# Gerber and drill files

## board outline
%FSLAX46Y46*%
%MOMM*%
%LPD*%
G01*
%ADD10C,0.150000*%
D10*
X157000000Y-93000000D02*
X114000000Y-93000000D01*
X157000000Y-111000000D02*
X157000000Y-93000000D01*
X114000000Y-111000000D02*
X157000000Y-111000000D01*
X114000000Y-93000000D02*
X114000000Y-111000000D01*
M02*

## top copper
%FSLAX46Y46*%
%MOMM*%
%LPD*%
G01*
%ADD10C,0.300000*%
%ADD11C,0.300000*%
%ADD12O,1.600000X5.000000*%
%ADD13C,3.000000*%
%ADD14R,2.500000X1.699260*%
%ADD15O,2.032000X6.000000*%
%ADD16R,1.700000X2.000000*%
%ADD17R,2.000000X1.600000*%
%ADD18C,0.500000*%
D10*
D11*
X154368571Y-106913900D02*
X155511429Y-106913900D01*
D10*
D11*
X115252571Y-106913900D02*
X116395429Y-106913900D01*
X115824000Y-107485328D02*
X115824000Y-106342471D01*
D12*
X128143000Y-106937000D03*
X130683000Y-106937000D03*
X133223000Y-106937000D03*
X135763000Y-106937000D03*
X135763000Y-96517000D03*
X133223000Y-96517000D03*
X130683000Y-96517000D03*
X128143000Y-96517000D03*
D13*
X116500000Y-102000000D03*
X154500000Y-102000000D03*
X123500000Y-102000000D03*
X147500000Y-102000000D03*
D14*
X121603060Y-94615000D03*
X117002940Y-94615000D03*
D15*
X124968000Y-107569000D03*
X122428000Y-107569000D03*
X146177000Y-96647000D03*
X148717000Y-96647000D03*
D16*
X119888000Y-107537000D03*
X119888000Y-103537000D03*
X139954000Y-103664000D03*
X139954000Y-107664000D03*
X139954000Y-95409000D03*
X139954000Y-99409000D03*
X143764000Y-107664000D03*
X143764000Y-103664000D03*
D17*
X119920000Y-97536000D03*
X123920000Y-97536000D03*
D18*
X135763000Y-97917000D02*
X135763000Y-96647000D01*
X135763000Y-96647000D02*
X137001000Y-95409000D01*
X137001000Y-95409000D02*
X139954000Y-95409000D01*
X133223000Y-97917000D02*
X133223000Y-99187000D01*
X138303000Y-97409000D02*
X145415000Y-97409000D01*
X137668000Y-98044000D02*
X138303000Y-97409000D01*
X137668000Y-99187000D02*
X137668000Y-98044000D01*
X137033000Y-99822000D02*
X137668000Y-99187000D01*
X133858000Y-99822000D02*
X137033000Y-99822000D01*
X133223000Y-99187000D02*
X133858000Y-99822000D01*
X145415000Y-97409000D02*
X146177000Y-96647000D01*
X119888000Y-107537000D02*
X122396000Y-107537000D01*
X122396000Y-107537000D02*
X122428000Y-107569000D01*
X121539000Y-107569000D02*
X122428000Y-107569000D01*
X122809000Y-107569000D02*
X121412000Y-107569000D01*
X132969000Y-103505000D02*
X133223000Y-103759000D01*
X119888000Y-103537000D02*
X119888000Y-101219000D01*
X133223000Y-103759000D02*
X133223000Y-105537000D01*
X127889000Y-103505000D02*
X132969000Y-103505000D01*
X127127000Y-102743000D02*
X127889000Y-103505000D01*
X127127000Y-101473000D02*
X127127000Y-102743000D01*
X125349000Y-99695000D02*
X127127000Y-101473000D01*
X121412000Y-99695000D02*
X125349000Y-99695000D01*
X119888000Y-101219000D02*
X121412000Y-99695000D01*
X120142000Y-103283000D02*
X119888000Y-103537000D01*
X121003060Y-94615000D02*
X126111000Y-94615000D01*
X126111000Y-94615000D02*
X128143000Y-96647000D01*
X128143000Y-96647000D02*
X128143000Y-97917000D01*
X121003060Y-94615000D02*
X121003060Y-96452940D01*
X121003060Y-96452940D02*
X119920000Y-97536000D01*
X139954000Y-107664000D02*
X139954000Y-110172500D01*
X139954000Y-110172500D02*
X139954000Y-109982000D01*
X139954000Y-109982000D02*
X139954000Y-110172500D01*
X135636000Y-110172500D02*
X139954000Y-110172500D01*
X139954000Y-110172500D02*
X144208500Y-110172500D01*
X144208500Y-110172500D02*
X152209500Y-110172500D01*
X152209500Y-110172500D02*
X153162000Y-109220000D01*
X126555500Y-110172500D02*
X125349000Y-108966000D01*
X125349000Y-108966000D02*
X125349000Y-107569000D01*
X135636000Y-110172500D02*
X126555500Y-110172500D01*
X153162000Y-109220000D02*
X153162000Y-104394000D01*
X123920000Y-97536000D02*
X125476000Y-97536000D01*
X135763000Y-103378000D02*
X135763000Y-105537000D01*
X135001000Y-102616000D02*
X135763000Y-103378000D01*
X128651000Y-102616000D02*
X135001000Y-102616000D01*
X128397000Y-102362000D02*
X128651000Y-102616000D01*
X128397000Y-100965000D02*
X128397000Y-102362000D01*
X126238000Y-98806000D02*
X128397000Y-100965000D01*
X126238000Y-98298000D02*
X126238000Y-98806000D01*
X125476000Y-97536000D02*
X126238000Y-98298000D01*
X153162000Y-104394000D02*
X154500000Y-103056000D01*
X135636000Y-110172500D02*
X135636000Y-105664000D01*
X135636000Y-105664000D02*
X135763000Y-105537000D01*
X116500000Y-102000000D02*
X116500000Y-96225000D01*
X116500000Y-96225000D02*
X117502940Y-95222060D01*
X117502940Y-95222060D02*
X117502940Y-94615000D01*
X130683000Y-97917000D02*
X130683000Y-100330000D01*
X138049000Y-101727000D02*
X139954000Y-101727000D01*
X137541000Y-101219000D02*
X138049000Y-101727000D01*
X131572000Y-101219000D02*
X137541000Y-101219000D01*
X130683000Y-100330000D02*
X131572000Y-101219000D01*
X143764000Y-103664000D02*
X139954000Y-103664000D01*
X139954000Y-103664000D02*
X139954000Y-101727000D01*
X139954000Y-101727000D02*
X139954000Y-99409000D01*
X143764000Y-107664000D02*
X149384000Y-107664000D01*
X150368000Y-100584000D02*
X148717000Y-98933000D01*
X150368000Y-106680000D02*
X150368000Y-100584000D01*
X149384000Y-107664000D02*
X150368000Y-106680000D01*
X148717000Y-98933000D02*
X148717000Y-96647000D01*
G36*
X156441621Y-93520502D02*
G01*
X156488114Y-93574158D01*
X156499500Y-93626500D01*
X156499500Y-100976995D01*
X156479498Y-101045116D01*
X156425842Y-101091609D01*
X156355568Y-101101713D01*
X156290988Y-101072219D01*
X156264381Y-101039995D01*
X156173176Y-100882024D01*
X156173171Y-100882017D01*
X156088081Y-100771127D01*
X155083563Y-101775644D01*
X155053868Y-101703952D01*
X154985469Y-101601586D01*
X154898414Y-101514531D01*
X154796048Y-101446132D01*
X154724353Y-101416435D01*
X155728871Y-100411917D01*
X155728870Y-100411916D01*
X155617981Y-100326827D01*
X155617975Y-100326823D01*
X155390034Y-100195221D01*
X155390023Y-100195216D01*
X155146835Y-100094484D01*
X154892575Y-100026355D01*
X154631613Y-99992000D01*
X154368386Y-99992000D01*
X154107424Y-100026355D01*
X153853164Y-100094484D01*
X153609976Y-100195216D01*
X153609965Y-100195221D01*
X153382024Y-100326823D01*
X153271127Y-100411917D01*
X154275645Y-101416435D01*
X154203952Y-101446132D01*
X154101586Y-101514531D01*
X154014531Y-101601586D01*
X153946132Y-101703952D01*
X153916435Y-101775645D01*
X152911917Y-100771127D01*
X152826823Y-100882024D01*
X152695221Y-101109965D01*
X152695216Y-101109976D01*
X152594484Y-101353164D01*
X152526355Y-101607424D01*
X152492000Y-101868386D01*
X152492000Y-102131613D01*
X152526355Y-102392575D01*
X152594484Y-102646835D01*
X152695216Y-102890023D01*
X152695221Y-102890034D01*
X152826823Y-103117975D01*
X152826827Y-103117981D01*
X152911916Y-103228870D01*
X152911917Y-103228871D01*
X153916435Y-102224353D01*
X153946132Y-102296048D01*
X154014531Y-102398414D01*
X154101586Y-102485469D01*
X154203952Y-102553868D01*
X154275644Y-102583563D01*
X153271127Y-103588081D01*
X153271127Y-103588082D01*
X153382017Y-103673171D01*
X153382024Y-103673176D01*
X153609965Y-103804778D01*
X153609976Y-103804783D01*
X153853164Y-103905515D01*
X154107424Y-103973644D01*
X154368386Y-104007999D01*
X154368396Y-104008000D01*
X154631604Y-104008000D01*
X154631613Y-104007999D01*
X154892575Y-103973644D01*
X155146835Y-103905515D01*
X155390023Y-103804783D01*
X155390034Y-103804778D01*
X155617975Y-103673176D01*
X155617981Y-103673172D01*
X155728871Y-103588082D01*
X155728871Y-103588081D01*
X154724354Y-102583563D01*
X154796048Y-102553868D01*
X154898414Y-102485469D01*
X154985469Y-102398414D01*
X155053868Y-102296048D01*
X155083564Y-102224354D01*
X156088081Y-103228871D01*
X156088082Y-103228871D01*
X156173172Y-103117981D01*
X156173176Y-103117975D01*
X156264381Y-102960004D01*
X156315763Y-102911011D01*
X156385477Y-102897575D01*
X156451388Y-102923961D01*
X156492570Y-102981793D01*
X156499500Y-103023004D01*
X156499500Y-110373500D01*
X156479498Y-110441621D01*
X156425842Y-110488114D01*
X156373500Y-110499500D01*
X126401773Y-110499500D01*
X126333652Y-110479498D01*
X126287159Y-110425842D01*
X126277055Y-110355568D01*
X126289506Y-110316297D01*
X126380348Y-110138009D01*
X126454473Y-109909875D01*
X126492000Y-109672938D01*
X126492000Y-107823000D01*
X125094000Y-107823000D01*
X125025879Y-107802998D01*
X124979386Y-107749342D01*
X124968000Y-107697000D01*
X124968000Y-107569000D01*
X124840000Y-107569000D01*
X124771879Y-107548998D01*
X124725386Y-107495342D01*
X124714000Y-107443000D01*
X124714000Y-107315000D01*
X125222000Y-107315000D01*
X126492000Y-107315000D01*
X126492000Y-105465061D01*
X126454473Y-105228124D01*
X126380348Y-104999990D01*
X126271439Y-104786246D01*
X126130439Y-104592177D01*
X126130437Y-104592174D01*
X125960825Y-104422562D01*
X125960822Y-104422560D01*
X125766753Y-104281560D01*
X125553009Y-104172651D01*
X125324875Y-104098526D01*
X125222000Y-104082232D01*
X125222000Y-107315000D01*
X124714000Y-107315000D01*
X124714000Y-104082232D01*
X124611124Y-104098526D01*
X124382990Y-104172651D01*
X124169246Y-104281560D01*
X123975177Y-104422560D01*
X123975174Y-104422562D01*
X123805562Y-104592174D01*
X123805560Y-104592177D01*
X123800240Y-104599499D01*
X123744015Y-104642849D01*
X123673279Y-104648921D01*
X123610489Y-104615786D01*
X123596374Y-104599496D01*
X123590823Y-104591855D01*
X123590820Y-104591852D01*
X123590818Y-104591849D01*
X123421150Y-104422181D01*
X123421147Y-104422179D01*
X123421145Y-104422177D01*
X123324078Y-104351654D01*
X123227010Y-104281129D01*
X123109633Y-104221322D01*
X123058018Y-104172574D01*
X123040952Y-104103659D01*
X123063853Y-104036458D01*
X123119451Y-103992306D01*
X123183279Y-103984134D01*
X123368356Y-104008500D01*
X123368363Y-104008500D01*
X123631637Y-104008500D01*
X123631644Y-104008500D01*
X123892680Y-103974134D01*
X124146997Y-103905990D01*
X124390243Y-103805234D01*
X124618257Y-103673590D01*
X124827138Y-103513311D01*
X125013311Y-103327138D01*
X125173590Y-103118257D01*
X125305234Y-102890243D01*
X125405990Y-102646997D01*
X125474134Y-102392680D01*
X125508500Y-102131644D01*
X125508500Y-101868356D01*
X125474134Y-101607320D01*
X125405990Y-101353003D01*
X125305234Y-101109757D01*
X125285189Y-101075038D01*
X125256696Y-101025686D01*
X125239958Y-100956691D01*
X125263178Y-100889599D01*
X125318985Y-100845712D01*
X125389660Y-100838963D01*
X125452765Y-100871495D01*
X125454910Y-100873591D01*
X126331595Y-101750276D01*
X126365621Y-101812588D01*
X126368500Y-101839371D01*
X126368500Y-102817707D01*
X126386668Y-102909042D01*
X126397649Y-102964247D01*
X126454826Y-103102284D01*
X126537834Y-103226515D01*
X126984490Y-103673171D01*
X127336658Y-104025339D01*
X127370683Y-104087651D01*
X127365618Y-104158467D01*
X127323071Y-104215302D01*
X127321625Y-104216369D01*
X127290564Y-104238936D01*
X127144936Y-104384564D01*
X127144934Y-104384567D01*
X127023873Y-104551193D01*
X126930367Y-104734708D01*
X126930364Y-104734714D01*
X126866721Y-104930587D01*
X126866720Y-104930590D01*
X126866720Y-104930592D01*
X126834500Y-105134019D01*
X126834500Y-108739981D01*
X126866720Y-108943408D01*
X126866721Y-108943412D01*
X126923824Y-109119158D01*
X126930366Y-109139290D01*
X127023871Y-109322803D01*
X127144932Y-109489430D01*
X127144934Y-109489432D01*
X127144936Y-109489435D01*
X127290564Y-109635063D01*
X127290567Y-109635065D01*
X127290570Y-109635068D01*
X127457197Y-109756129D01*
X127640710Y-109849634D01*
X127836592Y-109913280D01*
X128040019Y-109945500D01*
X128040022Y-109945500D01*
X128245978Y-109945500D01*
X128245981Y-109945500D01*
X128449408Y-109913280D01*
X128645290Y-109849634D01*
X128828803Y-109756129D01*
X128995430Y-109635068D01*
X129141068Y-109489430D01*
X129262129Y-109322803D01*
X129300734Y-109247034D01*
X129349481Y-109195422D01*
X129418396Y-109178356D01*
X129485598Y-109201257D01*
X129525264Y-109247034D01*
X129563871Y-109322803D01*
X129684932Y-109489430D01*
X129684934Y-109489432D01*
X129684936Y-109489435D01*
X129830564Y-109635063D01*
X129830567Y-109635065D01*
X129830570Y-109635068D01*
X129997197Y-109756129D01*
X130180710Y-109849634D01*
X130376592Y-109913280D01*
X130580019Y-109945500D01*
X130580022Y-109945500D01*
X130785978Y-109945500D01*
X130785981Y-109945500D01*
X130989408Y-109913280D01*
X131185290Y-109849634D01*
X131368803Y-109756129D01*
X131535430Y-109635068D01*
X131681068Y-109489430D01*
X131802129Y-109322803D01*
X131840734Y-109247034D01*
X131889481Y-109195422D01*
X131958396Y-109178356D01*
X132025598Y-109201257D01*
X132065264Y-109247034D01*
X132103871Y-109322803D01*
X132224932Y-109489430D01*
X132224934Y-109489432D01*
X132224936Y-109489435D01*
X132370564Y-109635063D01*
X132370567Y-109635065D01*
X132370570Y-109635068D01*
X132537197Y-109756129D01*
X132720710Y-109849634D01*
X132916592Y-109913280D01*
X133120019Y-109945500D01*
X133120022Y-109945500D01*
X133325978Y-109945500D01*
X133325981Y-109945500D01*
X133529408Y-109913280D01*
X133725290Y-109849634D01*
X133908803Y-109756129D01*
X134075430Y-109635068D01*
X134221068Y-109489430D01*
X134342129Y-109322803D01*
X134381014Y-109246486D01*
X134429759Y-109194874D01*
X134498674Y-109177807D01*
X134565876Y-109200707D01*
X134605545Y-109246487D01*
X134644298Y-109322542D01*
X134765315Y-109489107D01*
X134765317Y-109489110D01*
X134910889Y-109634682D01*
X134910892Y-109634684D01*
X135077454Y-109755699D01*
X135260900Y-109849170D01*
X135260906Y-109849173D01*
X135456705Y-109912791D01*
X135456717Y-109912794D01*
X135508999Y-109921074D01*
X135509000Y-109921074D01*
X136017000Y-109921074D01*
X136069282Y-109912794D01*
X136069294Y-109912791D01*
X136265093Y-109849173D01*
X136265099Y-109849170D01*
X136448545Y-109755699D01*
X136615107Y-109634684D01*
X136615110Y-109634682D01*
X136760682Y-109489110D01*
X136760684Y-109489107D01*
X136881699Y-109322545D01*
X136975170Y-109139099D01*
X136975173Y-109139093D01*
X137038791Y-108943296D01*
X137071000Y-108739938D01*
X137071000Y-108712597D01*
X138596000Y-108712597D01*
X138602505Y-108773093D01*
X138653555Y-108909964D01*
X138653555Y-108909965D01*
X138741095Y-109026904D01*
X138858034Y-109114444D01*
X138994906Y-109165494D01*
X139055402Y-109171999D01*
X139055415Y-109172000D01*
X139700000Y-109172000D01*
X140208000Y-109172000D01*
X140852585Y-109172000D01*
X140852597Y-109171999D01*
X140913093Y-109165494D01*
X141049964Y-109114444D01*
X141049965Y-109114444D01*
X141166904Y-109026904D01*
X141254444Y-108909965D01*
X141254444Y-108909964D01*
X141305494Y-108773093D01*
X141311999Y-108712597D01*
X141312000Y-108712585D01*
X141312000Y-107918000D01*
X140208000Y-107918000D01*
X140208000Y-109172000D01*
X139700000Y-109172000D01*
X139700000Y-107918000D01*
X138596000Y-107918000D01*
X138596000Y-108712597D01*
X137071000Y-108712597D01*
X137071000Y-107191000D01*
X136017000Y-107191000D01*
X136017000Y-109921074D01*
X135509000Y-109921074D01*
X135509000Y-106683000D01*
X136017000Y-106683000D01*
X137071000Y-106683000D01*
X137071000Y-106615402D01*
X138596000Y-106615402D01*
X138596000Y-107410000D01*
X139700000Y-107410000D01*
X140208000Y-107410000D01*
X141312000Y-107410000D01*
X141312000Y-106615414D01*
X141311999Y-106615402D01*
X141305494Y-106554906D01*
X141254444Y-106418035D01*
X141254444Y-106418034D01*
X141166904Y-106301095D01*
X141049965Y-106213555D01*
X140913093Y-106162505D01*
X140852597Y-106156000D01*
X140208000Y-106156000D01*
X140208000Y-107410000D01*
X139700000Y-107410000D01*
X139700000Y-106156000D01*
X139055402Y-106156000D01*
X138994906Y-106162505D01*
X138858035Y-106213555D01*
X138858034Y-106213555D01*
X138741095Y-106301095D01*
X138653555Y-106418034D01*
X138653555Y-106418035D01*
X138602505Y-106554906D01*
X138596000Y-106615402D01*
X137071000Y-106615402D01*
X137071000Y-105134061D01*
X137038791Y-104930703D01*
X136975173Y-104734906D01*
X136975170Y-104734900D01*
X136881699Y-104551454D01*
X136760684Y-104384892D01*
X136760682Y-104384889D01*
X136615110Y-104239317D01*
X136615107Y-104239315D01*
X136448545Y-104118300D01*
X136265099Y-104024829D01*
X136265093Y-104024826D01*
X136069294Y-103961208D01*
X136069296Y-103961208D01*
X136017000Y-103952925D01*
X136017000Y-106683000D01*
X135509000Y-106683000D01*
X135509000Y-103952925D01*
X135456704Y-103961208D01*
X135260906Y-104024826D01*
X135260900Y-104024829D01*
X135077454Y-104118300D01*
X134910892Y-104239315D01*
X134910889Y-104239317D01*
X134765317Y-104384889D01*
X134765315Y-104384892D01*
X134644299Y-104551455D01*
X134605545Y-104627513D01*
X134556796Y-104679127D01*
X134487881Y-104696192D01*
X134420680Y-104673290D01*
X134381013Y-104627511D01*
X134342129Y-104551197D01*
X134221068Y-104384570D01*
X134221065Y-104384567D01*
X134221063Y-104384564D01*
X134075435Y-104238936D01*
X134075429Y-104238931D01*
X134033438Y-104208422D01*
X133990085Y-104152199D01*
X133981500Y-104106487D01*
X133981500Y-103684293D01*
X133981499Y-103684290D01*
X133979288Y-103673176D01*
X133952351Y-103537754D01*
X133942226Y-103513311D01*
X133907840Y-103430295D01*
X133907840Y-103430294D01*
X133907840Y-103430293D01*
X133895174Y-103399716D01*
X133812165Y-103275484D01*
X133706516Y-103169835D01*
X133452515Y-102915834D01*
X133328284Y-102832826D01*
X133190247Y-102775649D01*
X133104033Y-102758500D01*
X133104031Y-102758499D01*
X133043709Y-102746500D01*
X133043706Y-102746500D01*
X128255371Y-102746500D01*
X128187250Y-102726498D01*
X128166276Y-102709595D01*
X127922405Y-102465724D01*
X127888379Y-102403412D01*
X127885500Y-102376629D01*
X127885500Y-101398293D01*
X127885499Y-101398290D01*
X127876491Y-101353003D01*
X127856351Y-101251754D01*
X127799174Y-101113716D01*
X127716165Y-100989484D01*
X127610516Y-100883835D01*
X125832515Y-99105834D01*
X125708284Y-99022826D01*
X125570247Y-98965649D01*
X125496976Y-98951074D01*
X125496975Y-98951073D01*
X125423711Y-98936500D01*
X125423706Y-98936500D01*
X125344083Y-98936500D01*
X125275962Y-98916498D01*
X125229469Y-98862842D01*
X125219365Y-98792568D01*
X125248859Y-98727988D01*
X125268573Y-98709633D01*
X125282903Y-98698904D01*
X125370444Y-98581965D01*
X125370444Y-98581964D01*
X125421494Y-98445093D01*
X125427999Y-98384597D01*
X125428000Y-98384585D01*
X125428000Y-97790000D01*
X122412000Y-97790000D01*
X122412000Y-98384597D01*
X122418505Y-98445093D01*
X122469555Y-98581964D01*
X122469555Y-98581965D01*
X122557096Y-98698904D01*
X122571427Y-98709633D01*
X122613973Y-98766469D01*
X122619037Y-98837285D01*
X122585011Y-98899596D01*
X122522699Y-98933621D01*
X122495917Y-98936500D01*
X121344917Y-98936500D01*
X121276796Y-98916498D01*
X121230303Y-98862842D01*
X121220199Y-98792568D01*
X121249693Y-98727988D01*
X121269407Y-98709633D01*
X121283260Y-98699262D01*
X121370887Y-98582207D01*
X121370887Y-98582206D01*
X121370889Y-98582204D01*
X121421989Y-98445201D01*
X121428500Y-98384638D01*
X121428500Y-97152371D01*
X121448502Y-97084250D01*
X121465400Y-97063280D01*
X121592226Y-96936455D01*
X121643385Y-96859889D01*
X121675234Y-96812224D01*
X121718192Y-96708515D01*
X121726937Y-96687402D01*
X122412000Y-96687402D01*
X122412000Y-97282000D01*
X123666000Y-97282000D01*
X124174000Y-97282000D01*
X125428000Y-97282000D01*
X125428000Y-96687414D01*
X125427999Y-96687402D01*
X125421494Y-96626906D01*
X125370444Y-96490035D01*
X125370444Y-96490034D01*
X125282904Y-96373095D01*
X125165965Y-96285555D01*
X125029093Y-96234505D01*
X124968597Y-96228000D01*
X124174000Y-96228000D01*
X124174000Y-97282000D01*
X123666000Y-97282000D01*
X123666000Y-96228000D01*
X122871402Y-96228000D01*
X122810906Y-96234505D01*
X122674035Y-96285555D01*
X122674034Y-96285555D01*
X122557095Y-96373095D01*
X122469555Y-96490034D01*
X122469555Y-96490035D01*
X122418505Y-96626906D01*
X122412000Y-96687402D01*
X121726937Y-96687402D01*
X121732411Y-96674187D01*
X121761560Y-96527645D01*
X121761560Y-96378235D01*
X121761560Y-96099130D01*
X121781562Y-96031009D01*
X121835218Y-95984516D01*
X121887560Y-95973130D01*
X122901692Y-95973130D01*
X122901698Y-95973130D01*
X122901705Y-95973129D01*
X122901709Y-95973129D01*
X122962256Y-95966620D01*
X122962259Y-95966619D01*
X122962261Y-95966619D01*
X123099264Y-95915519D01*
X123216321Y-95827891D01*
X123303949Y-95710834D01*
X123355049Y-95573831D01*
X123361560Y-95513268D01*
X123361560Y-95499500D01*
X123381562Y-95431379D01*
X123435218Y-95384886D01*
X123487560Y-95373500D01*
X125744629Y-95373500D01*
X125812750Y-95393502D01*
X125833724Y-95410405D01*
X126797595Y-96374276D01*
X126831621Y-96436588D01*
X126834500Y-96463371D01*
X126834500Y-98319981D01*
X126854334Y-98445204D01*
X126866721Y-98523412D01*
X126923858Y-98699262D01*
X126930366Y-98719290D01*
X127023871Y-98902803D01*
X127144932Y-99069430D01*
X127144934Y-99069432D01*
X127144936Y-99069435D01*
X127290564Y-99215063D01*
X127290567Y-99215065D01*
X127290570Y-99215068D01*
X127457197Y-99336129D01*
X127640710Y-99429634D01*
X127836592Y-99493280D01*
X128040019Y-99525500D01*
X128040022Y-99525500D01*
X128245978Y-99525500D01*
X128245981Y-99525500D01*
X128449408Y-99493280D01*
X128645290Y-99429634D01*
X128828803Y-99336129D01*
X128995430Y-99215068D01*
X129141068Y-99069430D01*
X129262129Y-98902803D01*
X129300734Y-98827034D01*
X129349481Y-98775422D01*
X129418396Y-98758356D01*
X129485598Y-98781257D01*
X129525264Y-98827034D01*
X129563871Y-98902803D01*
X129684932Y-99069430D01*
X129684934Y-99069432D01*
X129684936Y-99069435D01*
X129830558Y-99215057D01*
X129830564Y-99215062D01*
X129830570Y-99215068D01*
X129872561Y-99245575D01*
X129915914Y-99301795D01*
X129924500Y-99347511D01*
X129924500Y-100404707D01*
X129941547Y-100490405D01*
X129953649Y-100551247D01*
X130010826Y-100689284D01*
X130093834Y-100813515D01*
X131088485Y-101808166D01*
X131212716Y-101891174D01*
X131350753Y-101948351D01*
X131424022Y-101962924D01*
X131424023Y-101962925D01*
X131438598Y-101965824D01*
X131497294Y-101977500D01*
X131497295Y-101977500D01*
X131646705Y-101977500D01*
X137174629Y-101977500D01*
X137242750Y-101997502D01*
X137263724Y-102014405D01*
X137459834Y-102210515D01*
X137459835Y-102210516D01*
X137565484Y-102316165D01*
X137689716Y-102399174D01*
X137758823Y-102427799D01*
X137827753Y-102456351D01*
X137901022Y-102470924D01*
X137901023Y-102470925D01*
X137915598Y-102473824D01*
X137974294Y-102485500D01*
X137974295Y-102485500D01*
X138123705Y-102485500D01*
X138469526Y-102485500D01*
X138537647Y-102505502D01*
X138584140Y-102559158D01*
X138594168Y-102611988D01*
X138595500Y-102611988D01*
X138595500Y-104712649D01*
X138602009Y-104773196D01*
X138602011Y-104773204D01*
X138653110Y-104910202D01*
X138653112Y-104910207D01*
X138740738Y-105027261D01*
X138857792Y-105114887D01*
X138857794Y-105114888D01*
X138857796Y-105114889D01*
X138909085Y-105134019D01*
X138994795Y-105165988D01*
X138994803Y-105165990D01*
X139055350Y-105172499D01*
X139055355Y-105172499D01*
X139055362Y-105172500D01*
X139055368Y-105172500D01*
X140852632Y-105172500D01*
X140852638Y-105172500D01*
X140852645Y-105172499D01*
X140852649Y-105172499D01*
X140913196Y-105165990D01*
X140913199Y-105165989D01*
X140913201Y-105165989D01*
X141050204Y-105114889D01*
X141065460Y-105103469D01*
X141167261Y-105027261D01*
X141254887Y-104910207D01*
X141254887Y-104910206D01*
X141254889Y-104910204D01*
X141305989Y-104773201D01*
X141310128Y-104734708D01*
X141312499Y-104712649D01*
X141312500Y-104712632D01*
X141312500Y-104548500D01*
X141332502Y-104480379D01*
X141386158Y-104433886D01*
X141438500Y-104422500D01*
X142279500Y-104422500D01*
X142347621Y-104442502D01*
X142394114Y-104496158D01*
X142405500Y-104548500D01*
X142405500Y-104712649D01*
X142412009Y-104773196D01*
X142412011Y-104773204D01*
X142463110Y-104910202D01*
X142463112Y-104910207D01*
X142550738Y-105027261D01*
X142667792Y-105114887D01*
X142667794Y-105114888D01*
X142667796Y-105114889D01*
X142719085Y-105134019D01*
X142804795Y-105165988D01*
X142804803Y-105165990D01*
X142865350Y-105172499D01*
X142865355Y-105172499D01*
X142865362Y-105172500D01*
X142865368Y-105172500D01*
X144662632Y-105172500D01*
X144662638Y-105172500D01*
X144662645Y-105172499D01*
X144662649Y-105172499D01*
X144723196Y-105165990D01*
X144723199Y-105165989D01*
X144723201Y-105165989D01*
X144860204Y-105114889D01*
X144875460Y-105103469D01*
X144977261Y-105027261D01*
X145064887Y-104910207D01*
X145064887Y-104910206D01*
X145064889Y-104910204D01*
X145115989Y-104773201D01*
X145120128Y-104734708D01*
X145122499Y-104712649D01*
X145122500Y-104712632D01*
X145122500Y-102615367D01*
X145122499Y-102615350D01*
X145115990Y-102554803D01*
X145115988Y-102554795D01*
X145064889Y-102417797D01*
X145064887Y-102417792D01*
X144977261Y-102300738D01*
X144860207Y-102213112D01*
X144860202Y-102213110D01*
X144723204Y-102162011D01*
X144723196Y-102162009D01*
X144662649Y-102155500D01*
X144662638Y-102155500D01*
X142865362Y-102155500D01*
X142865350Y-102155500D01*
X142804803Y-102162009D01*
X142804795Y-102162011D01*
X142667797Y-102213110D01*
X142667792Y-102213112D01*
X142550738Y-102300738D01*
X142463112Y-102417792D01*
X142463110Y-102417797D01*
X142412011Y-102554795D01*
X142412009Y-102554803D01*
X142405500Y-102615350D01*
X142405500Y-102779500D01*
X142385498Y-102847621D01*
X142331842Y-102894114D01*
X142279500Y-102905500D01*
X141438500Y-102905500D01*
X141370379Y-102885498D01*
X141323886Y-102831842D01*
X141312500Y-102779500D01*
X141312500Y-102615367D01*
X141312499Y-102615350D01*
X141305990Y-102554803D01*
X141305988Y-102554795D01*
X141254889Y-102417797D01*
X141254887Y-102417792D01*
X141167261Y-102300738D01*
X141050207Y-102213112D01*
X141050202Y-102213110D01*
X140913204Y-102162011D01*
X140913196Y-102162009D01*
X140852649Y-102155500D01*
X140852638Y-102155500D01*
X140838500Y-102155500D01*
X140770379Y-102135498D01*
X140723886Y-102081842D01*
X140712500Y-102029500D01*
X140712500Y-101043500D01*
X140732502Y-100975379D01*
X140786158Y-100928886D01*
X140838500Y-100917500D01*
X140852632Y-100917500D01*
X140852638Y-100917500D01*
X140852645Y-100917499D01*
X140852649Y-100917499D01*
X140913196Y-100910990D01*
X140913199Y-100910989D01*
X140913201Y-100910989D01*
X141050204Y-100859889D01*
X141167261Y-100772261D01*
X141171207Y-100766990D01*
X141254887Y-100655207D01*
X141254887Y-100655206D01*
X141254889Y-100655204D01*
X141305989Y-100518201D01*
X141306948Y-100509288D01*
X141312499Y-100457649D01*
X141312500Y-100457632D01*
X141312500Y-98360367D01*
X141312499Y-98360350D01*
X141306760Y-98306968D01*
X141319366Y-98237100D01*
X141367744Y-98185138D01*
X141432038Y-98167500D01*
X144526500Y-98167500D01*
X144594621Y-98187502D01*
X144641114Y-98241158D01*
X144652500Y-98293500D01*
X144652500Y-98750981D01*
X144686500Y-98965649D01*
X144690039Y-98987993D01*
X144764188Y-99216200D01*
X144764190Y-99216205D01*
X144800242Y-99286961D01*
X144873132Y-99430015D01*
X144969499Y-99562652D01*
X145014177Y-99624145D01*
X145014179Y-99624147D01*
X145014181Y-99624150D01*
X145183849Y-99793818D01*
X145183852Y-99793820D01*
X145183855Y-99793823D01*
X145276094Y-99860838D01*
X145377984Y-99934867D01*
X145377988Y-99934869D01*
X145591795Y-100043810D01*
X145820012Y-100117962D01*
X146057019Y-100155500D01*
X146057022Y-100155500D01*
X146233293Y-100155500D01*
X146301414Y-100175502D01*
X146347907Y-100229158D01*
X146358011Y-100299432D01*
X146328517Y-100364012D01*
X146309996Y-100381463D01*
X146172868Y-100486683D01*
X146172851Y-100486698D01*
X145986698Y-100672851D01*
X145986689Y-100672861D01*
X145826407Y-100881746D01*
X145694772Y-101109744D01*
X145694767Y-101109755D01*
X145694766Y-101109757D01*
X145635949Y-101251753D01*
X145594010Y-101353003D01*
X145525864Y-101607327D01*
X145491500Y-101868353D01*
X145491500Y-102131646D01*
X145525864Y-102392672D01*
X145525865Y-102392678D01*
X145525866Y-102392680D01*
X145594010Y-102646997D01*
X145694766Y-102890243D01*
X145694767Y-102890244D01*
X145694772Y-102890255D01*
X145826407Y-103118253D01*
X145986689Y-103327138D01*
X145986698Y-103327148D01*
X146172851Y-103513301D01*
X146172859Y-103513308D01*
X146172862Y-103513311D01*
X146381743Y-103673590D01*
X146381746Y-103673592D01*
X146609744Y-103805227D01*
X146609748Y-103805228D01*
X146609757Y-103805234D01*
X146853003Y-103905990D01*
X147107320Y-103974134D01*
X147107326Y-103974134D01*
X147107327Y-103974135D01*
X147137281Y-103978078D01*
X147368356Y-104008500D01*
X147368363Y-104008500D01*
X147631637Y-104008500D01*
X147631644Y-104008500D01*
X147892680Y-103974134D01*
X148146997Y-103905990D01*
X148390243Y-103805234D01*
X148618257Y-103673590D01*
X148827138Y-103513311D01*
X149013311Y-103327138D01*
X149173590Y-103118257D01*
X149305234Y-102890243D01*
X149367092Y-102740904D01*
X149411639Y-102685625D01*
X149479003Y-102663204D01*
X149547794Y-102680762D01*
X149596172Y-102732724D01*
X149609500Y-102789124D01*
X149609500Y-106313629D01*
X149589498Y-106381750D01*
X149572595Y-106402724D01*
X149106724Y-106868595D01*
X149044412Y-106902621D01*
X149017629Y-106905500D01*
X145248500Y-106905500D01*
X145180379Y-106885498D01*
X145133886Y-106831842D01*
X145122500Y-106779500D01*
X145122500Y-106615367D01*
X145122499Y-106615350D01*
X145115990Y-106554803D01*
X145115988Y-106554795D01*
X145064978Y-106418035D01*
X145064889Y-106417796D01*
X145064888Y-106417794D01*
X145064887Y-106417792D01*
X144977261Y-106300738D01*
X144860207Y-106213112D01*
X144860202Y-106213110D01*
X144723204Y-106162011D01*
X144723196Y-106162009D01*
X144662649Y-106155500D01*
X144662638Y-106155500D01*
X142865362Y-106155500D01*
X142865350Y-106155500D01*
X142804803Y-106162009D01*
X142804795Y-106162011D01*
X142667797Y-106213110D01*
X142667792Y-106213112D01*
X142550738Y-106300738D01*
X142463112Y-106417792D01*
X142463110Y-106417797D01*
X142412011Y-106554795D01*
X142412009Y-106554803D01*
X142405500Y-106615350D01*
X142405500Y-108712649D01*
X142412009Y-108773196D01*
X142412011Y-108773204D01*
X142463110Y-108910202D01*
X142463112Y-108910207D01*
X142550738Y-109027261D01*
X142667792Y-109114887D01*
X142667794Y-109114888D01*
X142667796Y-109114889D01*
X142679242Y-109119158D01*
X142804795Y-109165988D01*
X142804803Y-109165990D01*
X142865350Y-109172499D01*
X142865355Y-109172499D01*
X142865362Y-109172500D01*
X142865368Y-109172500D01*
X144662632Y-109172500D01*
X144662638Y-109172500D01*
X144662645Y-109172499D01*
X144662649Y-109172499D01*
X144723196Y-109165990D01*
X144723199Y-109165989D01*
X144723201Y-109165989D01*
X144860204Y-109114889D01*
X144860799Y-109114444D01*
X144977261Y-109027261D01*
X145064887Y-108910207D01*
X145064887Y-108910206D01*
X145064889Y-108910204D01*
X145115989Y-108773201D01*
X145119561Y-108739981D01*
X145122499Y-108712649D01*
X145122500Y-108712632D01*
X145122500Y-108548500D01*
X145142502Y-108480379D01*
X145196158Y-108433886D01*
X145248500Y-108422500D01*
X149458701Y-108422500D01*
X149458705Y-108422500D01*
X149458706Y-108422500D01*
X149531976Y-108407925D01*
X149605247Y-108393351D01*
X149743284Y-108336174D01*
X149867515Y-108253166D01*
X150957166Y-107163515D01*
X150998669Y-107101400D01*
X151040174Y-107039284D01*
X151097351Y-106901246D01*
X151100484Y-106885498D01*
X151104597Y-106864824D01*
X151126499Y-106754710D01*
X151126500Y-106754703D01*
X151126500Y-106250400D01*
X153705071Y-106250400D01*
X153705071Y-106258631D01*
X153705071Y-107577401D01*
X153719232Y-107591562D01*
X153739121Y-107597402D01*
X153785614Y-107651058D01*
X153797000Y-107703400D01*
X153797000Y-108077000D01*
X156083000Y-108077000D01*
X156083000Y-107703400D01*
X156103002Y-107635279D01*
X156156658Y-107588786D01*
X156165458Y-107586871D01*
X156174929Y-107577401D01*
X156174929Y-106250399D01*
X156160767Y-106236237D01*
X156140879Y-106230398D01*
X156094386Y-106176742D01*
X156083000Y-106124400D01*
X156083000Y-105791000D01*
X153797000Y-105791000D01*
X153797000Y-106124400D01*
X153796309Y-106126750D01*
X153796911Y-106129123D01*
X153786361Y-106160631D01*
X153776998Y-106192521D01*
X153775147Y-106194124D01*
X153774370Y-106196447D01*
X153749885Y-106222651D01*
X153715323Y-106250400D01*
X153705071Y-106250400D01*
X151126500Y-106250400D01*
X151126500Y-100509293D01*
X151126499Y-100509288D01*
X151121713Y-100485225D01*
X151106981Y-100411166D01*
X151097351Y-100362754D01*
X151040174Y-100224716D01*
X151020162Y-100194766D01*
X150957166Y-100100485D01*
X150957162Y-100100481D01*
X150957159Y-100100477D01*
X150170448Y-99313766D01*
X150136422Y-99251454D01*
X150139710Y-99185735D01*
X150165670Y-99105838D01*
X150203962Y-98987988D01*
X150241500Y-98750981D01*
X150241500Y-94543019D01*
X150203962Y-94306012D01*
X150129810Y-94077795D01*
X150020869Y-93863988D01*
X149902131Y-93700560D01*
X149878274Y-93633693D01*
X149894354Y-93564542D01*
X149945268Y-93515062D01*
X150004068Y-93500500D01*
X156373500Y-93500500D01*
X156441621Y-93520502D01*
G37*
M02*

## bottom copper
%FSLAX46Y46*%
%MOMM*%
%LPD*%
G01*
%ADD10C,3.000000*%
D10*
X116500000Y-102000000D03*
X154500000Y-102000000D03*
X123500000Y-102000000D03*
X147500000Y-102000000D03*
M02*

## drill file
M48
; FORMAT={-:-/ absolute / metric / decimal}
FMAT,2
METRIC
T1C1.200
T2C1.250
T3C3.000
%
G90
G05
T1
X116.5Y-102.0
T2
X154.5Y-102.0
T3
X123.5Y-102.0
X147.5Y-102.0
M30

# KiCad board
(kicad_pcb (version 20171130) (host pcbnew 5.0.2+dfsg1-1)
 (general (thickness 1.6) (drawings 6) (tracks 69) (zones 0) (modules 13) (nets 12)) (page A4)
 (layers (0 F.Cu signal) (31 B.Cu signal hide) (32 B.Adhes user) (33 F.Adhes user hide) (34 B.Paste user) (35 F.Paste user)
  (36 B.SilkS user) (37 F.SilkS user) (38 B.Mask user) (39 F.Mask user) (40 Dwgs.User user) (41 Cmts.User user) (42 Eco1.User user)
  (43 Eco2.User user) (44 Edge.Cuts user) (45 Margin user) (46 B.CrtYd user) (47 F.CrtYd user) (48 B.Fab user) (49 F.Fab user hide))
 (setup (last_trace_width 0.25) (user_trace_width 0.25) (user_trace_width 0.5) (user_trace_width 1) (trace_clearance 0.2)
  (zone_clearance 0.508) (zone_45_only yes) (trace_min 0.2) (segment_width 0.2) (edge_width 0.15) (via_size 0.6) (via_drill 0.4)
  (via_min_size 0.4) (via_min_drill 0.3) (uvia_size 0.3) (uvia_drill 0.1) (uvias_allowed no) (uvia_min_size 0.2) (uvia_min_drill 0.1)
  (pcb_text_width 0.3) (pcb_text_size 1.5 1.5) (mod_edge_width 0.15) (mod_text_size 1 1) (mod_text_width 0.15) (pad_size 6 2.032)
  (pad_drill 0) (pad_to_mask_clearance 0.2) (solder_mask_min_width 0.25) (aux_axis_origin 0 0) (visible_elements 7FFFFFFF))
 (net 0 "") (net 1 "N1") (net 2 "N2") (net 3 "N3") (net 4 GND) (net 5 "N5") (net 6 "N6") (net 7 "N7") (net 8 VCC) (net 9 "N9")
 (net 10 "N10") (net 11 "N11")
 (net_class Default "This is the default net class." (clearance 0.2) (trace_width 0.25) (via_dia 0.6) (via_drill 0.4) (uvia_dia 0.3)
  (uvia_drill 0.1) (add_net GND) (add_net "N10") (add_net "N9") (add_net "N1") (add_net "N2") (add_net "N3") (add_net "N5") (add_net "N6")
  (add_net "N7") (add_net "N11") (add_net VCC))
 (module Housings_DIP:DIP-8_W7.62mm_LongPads (layer F.Cu) (at 128.143 105.537 90)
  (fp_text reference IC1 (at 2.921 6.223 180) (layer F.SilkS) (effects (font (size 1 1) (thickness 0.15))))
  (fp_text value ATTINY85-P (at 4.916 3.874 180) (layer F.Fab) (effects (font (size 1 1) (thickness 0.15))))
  (pad 1 smd oval (at 0 0 90) (size 5 1.6) (drill (offset -1.4 0)) (layers F.Cu F.Paste F.Mask) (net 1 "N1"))
  (pad 2 smd oval (at 0 2.54 90) (size 5 1.6) (drill (offset -1.4 0)) (layers F.Cu F.Paste F.Mask) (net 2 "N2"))
  (pad 3 smd oval (at 0 5.08 90) (size 5 1.6) (drill (offset -1.4 0)) (layers F.Cu F.Paste F.Mask) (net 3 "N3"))
  (pad 4 smd oval (at 0 7.62 90) (size 5 1.6) (drill (offset -1.4 0)) (layers F.Cu F.Paste F.Mask) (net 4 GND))
  (pad 5 smd oval (at 7.62 7.62 90) (size 5 1.6) (drill (offset 1.4 0)) (layers F.Cu F.Paste F.Mask) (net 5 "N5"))
  (pad 6 smd oval (at 7.62 5.08 90) (size 5 1.6) (drill (offset 1.4 0)) (layers F.Cu F.Paste F.Mask) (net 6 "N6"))
  (pad 7 smd oval (at 7.62 2.54 90) (size 5 1.6) (drill (offset 1.4 0)) (layers F.Cu F.Paste F.Mask) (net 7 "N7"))
  (pad 8 smd oval (at 7.62 0 90) (size 5 1.6) (drill (offset 1.4 0)) (layers F.Cu F.Paste F.Mask) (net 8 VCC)))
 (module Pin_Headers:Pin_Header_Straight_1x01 (layer F.Cu) (at 116.5 102)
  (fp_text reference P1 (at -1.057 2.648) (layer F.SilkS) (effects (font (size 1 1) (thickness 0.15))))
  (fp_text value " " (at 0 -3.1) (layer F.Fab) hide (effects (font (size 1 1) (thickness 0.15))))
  (pad 1 thru_hole circle (at 0 0) (size 3 3) (drill 1.2) (layers F.Cu F.SilkS F.Mask) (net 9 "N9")))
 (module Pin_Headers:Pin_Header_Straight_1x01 (layer F.Cu) (at 154.5 102)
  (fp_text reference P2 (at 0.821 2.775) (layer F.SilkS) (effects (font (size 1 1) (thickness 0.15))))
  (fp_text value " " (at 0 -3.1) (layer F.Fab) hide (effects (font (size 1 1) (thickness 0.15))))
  (pad 1 thru_hole circle (at 0 0) (size 3 3) (drill 1.25) (layers *.Mask F.Cu F.SilkS) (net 4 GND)))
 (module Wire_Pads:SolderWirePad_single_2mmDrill (layer F.Cu) (at 123.5 102)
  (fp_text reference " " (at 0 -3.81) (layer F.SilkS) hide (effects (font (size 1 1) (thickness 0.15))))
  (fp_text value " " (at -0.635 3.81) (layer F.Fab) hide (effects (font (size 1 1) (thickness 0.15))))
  (pad 1 thru_hole circle (at 0 0) (size 3 3) (drill 3) (layers *.Mask F.Cu F.SilkS)))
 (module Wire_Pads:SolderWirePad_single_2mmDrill (layer F.Cu) (at 147.5 102)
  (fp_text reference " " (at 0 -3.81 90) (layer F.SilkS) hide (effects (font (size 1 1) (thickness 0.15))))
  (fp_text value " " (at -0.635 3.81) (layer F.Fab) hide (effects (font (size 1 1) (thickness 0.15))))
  (pad 1 thru_hole circle (at 0 0) (size 3 3) (drill 3) (layers *.Mask F.Cu F.SilkS)))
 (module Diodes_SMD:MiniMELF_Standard (layer F.Cu) (at 119.253 94.615 180)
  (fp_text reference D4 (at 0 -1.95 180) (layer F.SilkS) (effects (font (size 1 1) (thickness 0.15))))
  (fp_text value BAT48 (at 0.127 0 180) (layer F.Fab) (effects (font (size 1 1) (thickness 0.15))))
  (pad 1 smd rect (at -1.75006 0 180) (size 2.5 1.69926) (drill (offset -0.6 0)) (layers F.Cu F.Paste F.Mask) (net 8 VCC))
  (pad 2 smd rect (at 1.75006 0 180) (size 2.5 1.69926) (drill (offset 0.5 0)) (layers F.Cu F.Paste F.Mask) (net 9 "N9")))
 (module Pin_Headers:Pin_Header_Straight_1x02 (layer F.Cu) (at 124.968 107.569 270)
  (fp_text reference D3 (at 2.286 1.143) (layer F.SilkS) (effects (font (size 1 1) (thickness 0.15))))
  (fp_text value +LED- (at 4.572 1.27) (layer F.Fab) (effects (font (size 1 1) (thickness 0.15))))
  (pad 1 smd oval (at 0 0 270) (size 6 2.032) (layers F.Cu F.Paste F.Mask) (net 4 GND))
  (pad 2 smd oval (at 0 2.54 270) (size 6 2.032) (layers F.Cu F.Paste F.Mask) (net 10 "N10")))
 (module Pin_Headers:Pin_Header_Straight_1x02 (layer F.Cu) (at 146.177 96.647 90)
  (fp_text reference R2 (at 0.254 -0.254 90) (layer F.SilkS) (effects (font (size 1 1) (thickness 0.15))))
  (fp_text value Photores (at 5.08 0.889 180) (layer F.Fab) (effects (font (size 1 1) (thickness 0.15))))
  (pad 1 smd oval (at 0 0 90) (size 6 2.032) (layers F.Cu F.Paste F.Mask) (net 6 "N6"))
  (pad 2 smd oval (at 0 2.54 90) (size 6 2.032) (layers F.Cu F.Paste F.Mask) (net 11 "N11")))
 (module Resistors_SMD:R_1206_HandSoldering (layer F.Cu) (at 119.888 105.537 90)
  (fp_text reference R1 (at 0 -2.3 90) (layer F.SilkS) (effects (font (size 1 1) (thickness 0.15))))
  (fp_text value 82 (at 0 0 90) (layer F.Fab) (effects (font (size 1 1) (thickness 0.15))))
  (pad 1 smd rect (at -2 0 90) (size 2 1.7) (layers F.Cu F.Paste F.Mask) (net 10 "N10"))
  (pad 2 smd rect (at 2 0 90) (size 2 1.7) (layers F.Cu F.Paste F.Mask) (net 3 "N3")))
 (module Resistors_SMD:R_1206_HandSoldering (layer F.Cu) (at 139.954 105.664 270)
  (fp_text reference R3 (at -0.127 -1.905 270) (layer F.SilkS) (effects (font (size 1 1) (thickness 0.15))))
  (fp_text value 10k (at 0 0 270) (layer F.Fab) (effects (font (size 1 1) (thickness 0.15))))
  (pad 1 smd rect (at -2 0 270) (size 2 1.7) (layers F.Cu F.Paste F.Mask) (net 7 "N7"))
  (pad 2 smd rect (at 2 0 270) (size 2 1.7) (layers F.Cu F.Paste F.Mask) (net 4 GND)))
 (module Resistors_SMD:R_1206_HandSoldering (layer F.Cu) (at 139.954 97.409 270)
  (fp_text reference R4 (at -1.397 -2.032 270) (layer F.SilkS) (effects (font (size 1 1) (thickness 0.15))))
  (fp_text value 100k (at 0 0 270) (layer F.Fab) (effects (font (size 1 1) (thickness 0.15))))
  (pad 1 smd rect (at -2 0 270) (size 2 1.7) (layers F.Cu F.Paste F.Mask) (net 5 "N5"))
  (pad 2 smd rect (at 2 0 270) (size 2 1.7) (layers F.Cu F.Paste F.Mask) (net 7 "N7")))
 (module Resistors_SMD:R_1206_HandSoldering (layer F.Cu) (at 143.764 105.664 90)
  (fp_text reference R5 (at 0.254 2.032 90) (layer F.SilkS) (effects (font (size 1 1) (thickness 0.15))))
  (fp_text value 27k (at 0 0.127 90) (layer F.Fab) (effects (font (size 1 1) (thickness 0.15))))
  (pad 1 smd rect (at -2 0 90) (size 2 1.7) (layers F.Cu F.Paste F.Mask) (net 11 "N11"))
  (pad 2 smd rect (at 2 0 90) (size 2 1.7) (layers F.Cu F.Paste F.Mask) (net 7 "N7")))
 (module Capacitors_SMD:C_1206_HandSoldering (layer F.Cu) (at 121.92 97.536)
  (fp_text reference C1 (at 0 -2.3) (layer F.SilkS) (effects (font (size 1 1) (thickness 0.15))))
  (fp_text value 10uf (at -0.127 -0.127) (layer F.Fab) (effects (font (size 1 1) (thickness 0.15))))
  (pad 1 smd rect (at -2 0) (size 2 1.6) (layers F.Cu F.Paste F.Mask) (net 8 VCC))
  (pad 2 smd rect (at 2 0) (size 2 1.6) (layers F.Cu F.Paste F.Mask) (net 4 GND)))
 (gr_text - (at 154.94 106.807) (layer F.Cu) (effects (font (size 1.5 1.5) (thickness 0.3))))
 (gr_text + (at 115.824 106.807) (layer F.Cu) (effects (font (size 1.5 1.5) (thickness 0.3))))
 (gr_line (start 157 93) (end 114 93) (angle 90) (layer Edge.Cuts) (width 0.15))
 (gr_line (start 157 111) (end 157 93) (angle 90) (layer Edge.Cuts) (width 0.15))
 (gr_line (start 114 111) (end 157 111) (angle 90) (layer Edge.Cuts) (width 0.15))
 (gr_line (start 114 93) (end 114 111) (angle 90) (layer Edge.Cuts) (width 0.15))
 (segment (start 135.763 97.917) (end 135.763 96.647) (width 0.5) (layer F.Cu) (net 5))
 (segment (start 135.763 96.647) (end 137.001 95.409) (width 0.5) (layer F.Cu) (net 5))
 (segment (start 137.001 95.409) (end 139.954 95.409) (width 0.5) (layer F.Cu) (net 5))
 (segment (start 133.223 97.917) (end 133.223 99.187) (width 0.5) (layer F.Cu) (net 6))
 (segment (start 138.303 97.409) (end 145.415 97.409) (width 0.5) (layer F.Cu) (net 6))
 (segment (start 137.668 98.044) (end 138.303 97.409) (width 0.5) (layer F.Cu) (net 6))
 (segment (start 137.668 99.187) (end 137.668 98.044) (width 0.5) (layer F.Cu) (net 6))
 (segment (start 137.033 99.822) (end 137.668 99.187) (width 0.5) (layer F.Cu) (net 6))
 (segment (start 133.858 99.822) (end 137.033 99.822) (width 0.5) (layer F.Cu) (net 6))
 (segment (start 133.223 99.187) (end 133.858 99.822) (width 0.5) (layer F.Cu) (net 6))
 (segment (start 145.415 97.409) (end 146.177 96.647) (width 0.5) (layer F.Cu) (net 6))
 (segment (start 119.888 107.537) (end 122.396 107.537) (width 0.5) (layer F.Cu) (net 10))
 (segment (start 122.396 107.537) (end 122.428 107.569) (width 0.5) (layer F.Cu) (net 10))
 (segment (start 121.539 107.569) (end 122.428 107.569) (width 0.5) (layer F.Cu) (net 10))
 (segment (start 122.809 107.569) (end 121.412 107.569) (width 0.5) (layer F.Cu) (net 10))
 (segment (start 132.969 103.505) (end 133.223 103.759) (width 0.5) (layer F.Cu) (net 3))
 (segment (start 119.888 103.537) (end 119.888 101.219) (width 0.5) (layer F.Cu) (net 3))
 (segment (start 133.223 103.759) (end 133.223 105.537) (width 0.5) (layer F.Cu) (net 3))
 (segment (start 127.889 103.505) (end 132.969 103.505) (width 0.5) (layer F.Cu) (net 3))
 (segment (start 127.127 102.743) (end 127.889 103.505) (width 0.5) (layer F.Cu) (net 3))
 (segment (start 127.127 101.473) (end 127.127 102.743) (width 0.5) (layer F.Cu) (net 3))
 (segment (start 125.349 99.695) (end 127.127 101.473) (width 0.5) (layer F.Cu) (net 3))
 (segment (start 121.412 99.695) (end 125.349 99.695) (width 0.5) (layer F.Cu) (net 3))
 (segment (start 119.888 101.219) (end 121.412 99.695) (width 0.5) (layer F.Cu) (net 3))
 (segment (start 120.142 103.283) (end 119.888 103.537) (width 0.5) (layer F.Cu) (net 3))
 (segment (start 121.00306 94.615) (end 126.111 94.615) (width 0.5) (layer F.Cu) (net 8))
 (segment (start 126.111 94.615) (end 128.143 96.647) (width 0.5) (layer F.Cu) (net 8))
 (segment (start 128.143 96.647) (end 128.143 97.917) (width 0.5) (layer F.Cu) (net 8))
 (segment (start 121.00306 94.615) (end 121.00306 96.45294) (width 0.5) (layer F.Cu) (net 8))
 (segment (start 121.00306 96.45294) (end 119.92 97.536) (width 0.5) (layer F.Cu) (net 8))
 (segment (start 139.954 107.664) (end 139.954 110.1725) (width 0.5) (layer F.Cu) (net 4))
 (segment (start 139.954 110.1725) (end 139.954 109.982) (width 0.5) (layer F.Cu) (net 4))
 (segment (start 139.954 109.982) (end 139.954 110.1725) (width 0.5) (layer F.Cu) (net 4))
 (segment (start 135.636 110.1725) (end 139.954 110.1725) (width 0.5) (layer F.Cu) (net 4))
 (segment (start 139.954 110.1725) (end 144.2085 110.1725) (width 0.5) (layer F.Cu) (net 4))
 (segment (start 144.2085 110.1725) (end 152.2095 110.1725) (width 0.5) (layer F.Cu) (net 4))
 (segment (start 152.2095 110.1725) (end 153.162 109.22) (width 0.5) (layer F.Cu) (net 4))
 (segment (start 126.5555 110.1725) (end 125.349 108.966) (width 0.5) (layer F.Cu) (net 4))
 (segment (start 125.349 108.966) (end 125.349 107.569) (width 0.5) (layer F.Cu) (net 4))
 (segment (start 135.636 110.1725) (end 126.5555 110.1725) (width 0.5) (layer F.Cu) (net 4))
 (segment (start 153.162 109.22) (end 153.162 104.394) (width 0.5) (layer F.Cu) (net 4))
 (segment (start 123.92 97.536) (end 125.476 97.536) (width 0.5) (layer F.Cu) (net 4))
 (segment (start 135.763 103.378) (end 135.763 105.537) (width 0.5) (layer F.Cu) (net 4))
 (segment (start 135.001 102.616) (end 135.763 103.378) (width 0.5) (layer F.Cu) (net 4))
 (segment (start 128.651 102.616) (end 135.001 102.616) (width 0.5) (layer F.Cu) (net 4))
 (segment (start 128.397 102.362) (end 128.651 102.616) (width 0.5) (layer F.Cu) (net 4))
 (segment (start 128.397 100.965) (end 128.397 102.362) (width 0.5) (layer F.Cu) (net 4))
 (segment (start 126.238 98.806) (end 128.397 100.965) (width 0.5) (layer F.Cu) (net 4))
 (segment (start 126.238 98.298) (end 126.238 98.806) (width 0.5) (layer F.Cu) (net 4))
 (segment (start 125.476 97.536) (end 126.238 98.298) (width 0.5) (layer F.Cu) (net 4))
 (segment (start 153.162 104.394) (end 154.5 103.056) (width 0.5) (layer F.Cu) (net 4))
 (segment (start 135.636 110.1725) (end 135.636 105.664) (width 0.5) (layer F.Cu) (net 4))
 (segment (start 135.636 105.664) (end 135.763 105.537) (width 0.5) (layer F.Cu) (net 4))
 (segment (start 116.5 102) (end 116.5 96.225) (width 0.5) (layer F.Cu) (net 9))
 (segment (start 116.5 96.225) (end 117.50294 95.22206) (width 0.5) (layer F.Cu) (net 9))
 (segment (start 117.50294 95.22206) (end 117.50294 94.615) (width 0.5) (layer F.Cu) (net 9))
 (segment (start 130.683 97.917) (end 130.683 100.33) (width 0.5) (layer F.Cu) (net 7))
 (segment (start 138.049 101.727) (end 139.954 101.727) (width 0.5) (layer F.Cu) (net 7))
 (segment (start 137.541 101.219) (end 138.049 101.727) (width 0.5) (layer F.Cu) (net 7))
 (segment (start 131.572 101.219) (end 137.541 101.219) (width 0.5) (layer F.Cu) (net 7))
 (segment (start 130.683 100.33) (end 131.572 101.219) (width 0.5) (layer F.Cu) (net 7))
 (segment (start 143.764 103.664) (end 139.954 103.664) (width 0.5) (layer F.Cu) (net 7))
 (segment (start 139.954 103.664) (end 139.954 101.727) (width 0.5) (layer F.Cu) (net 7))
 (segment (start 139.954 101.727) (end 139.954 99.409) (width 0.5) (layer F.Cu) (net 7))
 (segment (start 143.764 107.664) (end 149.384 107.664) (width 0.5) (layer F.Cu) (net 11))
 (segment (start 150.368 100.584) (end 148.717 98.933) (width 0.5) (layer F.Cu) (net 11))
 (segment (start 150.368 106.68) (end 150.368 100.584) (width 0.5) (layer F.Cu) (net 11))
 (segment (start 149.384 107.664) (end 150.368 106.68) (width 0.5) (layer F.Cu) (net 11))
 (segment (start 148.717 98.933) (end 148.717 96.647) (width 0.5) (layer F.Cu) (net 11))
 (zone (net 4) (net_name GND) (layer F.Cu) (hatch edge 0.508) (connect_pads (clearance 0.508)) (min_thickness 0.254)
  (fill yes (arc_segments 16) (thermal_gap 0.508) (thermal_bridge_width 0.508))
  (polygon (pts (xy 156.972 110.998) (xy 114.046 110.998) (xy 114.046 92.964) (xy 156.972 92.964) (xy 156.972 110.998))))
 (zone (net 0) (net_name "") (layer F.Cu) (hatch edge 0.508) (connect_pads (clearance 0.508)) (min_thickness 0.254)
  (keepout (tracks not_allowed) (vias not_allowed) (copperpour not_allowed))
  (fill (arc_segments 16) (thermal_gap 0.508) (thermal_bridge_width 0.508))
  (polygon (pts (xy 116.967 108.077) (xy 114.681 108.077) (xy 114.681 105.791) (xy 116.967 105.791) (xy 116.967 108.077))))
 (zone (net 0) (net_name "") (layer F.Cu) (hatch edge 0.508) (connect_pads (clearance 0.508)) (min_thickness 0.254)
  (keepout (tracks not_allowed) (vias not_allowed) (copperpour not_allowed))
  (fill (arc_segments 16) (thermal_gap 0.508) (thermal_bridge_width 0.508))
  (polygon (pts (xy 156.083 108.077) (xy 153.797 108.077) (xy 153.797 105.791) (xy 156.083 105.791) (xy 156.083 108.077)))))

